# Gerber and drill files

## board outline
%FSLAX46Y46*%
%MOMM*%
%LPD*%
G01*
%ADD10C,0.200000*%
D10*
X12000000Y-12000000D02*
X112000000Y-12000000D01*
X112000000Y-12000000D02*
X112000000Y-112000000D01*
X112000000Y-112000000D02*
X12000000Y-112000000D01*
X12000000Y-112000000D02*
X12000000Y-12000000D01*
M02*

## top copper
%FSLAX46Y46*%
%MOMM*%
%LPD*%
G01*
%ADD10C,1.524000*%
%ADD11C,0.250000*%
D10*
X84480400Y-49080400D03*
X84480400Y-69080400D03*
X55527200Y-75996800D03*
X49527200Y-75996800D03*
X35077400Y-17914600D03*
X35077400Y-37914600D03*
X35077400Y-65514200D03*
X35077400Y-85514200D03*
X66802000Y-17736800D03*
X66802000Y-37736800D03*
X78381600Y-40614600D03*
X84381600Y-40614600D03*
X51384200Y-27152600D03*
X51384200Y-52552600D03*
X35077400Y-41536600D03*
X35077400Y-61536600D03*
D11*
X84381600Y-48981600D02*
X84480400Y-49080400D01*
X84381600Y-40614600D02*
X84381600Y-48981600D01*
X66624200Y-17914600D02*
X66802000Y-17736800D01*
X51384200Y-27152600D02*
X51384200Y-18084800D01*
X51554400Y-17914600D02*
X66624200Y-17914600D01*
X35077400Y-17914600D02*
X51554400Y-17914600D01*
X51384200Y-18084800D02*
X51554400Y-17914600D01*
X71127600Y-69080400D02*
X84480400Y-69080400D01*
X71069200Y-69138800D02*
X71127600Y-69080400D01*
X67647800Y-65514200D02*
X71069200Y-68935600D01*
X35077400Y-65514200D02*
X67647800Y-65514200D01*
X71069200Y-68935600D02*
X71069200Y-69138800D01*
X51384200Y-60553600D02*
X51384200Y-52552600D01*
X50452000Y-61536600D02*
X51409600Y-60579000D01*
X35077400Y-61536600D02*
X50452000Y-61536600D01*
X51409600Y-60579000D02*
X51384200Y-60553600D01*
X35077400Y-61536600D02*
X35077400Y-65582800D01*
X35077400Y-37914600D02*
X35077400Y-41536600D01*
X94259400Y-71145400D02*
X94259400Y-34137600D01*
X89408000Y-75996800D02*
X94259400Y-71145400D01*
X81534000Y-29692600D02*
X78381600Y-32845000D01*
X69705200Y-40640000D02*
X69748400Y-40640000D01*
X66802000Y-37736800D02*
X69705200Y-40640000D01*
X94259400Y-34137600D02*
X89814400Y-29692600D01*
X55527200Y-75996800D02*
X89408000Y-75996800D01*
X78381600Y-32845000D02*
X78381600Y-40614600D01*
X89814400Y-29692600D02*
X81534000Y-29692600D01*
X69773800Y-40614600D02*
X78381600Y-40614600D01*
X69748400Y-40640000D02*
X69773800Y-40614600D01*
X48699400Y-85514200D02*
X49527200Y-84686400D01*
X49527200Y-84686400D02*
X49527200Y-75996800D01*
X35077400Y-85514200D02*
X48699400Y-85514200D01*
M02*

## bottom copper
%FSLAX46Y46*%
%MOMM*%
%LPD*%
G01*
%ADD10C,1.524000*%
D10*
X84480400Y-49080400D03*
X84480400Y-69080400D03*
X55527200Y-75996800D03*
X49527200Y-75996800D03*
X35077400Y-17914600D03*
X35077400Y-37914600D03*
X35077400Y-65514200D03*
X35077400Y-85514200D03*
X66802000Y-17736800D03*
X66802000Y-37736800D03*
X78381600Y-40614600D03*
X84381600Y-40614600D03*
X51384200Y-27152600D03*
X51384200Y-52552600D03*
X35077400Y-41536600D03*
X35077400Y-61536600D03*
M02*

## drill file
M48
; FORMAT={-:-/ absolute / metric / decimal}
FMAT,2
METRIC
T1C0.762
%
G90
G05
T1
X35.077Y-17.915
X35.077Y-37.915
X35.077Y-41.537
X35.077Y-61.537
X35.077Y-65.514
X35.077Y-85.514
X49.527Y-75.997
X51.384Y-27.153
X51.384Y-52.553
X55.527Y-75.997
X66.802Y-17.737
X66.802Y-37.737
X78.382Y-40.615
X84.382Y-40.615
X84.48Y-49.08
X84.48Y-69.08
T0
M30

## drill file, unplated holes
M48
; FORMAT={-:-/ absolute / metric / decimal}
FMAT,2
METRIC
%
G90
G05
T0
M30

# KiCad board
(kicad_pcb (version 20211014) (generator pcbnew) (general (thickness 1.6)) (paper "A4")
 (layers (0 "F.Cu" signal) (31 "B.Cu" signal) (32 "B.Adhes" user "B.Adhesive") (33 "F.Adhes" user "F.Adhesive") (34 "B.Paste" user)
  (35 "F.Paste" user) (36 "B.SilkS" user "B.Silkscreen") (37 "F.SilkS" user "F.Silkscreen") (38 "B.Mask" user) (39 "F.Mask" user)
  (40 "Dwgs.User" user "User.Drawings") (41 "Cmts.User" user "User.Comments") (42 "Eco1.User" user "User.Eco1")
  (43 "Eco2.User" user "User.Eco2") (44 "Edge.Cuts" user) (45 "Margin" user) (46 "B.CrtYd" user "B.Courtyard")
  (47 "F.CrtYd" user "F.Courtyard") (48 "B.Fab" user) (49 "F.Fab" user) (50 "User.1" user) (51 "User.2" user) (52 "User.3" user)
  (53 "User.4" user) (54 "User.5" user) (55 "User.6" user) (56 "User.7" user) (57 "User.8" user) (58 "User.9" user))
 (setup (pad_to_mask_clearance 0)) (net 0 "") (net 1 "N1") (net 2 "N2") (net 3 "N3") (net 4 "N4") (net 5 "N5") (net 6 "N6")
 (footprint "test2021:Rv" (layer "F.Cu") (at 84.4804 59.0804 -90)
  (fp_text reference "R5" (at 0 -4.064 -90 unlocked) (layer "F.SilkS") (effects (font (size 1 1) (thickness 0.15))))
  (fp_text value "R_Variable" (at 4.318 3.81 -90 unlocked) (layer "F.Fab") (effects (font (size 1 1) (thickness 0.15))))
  (pad "1" thru_hole circle (at -10 0 270) (size 1.524 1.524) (drill 0.762) (layers *.Cu *.Mask) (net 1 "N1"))
  (pad "2" thru_hole circle (at 10 0 270) (size 1.524 1.524) (drill 0.762) (layers *.Cu *.Mask) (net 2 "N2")))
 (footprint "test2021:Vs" (layer "F.Cu") (at 52.5272 75.9968 -90)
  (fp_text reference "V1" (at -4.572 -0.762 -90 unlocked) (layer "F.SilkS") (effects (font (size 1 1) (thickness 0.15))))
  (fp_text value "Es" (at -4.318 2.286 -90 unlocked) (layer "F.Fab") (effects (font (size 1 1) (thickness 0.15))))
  (pad "1" thru_hole circle (at 0 -3 270) (size 1.524 1.524) (drill 0.762) (layers *.Cu *.Mask) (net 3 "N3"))
  (pad "2" thru_hole circle (at 0 3 270) (size 1.524 1.524) (drill 0.762) (layers *.Cu *.Mask) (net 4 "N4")))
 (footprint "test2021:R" (layer "F.Cu") (at 35.0774 27.9146 -90)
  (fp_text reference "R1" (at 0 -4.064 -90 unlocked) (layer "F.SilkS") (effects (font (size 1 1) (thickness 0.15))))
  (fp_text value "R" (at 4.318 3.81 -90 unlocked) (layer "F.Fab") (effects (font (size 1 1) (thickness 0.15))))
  (pad "1" thru_hole circle (at -10 0 270) (size 1.524 1.524) (drill 0.762) (layers *.Cu *.Mask) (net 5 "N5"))
  (pad "2" thru_hole circle (at 10 0 270) (size 1.524 1.524) (drill 0.762) (layers *.Cu *.Mask) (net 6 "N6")))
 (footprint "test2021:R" (layer "F.Cu") (at 35.0774 75.5142 -90)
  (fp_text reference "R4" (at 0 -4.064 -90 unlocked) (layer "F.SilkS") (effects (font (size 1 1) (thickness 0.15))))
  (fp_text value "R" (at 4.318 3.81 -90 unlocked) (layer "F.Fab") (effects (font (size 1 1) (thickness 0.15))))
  (pad "1" thru_hole circle (at -10 0 270) (size 1.524 1.524) (drill 0.762) (layers *.Cu *.Mask) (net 2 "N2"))
  (pad "2" thru_hole circle (at 10 0 270) (size 1.524 1.524) (drill 0.762) (layers *.Cu *.Mask) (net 4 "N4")))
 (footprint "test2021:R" (layer "F.Cu") (at 66.802 27.7368 -90)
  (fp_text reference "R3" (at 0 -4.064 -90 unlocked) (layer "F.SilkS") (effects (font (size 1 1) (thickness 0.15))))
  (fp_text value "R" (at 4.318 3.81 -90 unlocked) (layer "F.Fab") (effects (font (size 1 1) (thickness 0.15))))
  (pad "1" thru_hole circle (at -10 0 270) (size 1.524 1.524) (drill 0.762) (layers *.Cu *.Mask) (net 5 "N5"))
  (pad "2" thru_hole circle (at 10 0 270) (size 1.524 1.524) (drill 0.762) (layers *.Cu *.Mask) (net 3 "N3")))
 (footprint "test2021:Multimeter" (layer "F.Cu") (at 81.3816 40.6146 90)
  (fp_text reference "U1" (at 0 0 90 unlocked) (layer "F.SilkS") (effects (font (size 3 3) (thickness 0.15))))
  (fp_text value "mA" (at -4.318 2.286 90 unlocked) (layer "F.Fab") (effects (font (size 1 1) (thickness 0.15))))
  (pad "1" thru_hole circle (at 0 -3 90) (size 1.524 1.524) (drill 0.762) (layers *.Cu *.Mask) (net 3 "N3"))
  (pad "2" thru_hole circle (at 0 3 90) (size 1.524 1.524) (drill 0.762) (layers *.Cu *.Mask) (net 1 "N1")))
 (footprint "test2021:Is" (layer "F.Cu") (at 51.3842 39.8526 -90)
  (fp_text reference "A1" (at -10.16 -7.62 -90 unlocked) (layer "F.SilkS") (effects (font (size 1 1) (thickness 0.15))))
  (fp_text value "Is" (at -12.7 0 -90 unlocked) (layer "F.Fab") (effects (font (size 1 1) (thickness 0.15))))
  (pad "1" thru_hole circle (at -12.7 0 270) (size 1.524 1.524) (drill 0.762) (layers *.Cu *.Mask) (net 5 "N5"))
  (pad "2" thru_hole circle (at 12.7 0 270) (size 1.524 1.524) (drill 0.762) (layers *.Cu *.Mask) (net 2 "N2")))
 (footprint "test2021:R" (layer "F.Cu") (at 35.0774 51.5366 -90)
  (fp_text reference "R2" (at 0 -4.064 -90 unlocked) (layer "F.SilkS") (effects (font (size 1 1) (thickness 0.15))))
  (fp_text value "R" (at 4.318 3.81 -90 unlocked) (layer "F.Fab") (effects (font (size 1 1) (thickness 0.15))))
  (pad "1" thru_hole circle (at -10 0 270) (size 1.524 1.524) (drill 0.762) (layers *.Cu *.Mask) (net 6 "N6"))
  (pad "2" thru_hole circle (at 10 0 270) (size 1.524 1.524) (drill 0.762) (layers *.Cu *.Mask) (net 2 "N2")))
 (gr_rect (start 12 12) (end 112 112) (layer "Edge.Cuts") (width 0.2) (fill none))
 (segment (start 66.6242 17.9146) (end 66.802 17.7368) (width 0.25) (layer "F.Cu") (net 5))
 (segment (start 51.3842 27.1526) (end 51.3842 18.0848) (width 0.25) (layer "F.Cu") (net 5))
 (segment (start 51.5544 17.9146) (end 66.6242 17.9146) (width 0.25) (layer "F.Cu") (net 5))
 (segment (start 35.0774 17.9146) (end 51.5544 17.9146) (width 0.25) (layer "F.Cu") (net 5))
 (segment (start 51.3842 18.0848) (end 51.5544 17.9146) (width 0.25) (layer "F.Cu") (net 5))
 (segment (start 71.1276 69.0804) (end 84.4804 69.0804) (width 0.25) (layer "F.Cu") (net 2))
 (segment (start 71.0692 69.1388) (end 71.1276 69.0804) (width 0.25) (layer "F.Cu") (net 2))
 (segment (start 67.6478 65.5142) (end 71.0692 68.9356) (width 0.25) (layer "F.Cu") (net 2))
 (segment (start 35.0774 65.5142) (end 67.6478 65.5142) (width 0.25) (layer "F.Cu") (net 2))
 (segment (start 71.0692 68.9356) (end 71.0692 69.1388) (width 0.25) (layer "F.Cu") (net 2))
 (segment (start 51.3842 60.5536) (end 51.3842 52.5526) (width 0.25) (layer "F.Cu") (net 2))
 (segment (start 50.452 61.5366) (end 51.4096 60.579) (width 0.25) (layer "F.Cu") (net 2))
 (segment (start 35.0774 61.5366) (end 50.452 61.5366) (width 0.25) (layer "F.Cu") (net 2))
 (segment (start 51.4096 60.579) (end 51.3842 60.5536) (width 0.25) (layer "F.Cu") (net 2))
 (segment (start 35.0774 61.5366) (end 35.0774 65.5828) (width 0.25) (layer "F.Cu") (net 2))
 (segment (start 35.0774 37.9146) (end 35.0774 41.5366) (width 0.25) (layer "F.Cu") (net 6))
 (segment (start 94.2594 71.1454) (end 94.2594 34.1376) (width 0.25) (layer "F.Cu") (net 3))
 (segment (start 89.408 75.9968) (end 94.2594 71.1454) (width 0.25) (layer "F.Cu") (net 3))
 (segment (start 81.534 29.6926) (end 78.3816 32.845) (width 0.25) (layer "F.Cu") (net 3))
 (segment (start 69.7052 40.64) (end 69.7484 40.64) (width 0.25) (layer "F.Cu") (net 3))
 (segment (start 66.802 37.7368) (end 69.7052 40.64) (width 0.25) (layer "F.Cu") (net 3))
 (segment (start 94.2594 34.1376) (end 89.8144 29.6926) (width 0.25) (layer "F.Cu") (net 3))
 (segment (start 55.5272 75.9968) (end 89.408 75.9968) (width 0.25) (layer "F.Cu") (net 3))
 (segment (start 78.3816 32.845) (end 78.3816 40.6146) (width 0.25) (layer "F.Cu") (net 3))
 (segment (start 89.8144 29.6926) (end 81.534 29.6926) (width 0.25) (layer "F.Cu") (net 3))
 (segment (start 69.7738 40.6146) (end 78.3816 40.6146) (width 0.25) (layer "F.Cu") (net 3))
 (segment (start 69.7484 40.64) (end 69.7738 40.6146) (width 0.25) (layer "F.Cu") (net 3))
 (segment (start 48.6994 85.5142) (end 49.5272 84.6864) (width 0.25) (layer "F.Cu") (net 4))
 (segment (start 49.5272 84.6864) (end 49.5272 75.9968) (width 0.25) (layer "F.Cu") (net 4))
 (segment (start 35.0774 85.5142) (end 48.6994 85.5142) (width 0.25) (layer "F.Cu") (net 4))
 (segment (start 84.3816 40.6146) (end 84.3816 48.9816) (width 0.25) (layer "F.Cu") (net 1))
 (segment (start 84.3816 48.9816) (end 84.4804 49.0804) (width 0.25) (layer "F.Cu") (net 1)))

